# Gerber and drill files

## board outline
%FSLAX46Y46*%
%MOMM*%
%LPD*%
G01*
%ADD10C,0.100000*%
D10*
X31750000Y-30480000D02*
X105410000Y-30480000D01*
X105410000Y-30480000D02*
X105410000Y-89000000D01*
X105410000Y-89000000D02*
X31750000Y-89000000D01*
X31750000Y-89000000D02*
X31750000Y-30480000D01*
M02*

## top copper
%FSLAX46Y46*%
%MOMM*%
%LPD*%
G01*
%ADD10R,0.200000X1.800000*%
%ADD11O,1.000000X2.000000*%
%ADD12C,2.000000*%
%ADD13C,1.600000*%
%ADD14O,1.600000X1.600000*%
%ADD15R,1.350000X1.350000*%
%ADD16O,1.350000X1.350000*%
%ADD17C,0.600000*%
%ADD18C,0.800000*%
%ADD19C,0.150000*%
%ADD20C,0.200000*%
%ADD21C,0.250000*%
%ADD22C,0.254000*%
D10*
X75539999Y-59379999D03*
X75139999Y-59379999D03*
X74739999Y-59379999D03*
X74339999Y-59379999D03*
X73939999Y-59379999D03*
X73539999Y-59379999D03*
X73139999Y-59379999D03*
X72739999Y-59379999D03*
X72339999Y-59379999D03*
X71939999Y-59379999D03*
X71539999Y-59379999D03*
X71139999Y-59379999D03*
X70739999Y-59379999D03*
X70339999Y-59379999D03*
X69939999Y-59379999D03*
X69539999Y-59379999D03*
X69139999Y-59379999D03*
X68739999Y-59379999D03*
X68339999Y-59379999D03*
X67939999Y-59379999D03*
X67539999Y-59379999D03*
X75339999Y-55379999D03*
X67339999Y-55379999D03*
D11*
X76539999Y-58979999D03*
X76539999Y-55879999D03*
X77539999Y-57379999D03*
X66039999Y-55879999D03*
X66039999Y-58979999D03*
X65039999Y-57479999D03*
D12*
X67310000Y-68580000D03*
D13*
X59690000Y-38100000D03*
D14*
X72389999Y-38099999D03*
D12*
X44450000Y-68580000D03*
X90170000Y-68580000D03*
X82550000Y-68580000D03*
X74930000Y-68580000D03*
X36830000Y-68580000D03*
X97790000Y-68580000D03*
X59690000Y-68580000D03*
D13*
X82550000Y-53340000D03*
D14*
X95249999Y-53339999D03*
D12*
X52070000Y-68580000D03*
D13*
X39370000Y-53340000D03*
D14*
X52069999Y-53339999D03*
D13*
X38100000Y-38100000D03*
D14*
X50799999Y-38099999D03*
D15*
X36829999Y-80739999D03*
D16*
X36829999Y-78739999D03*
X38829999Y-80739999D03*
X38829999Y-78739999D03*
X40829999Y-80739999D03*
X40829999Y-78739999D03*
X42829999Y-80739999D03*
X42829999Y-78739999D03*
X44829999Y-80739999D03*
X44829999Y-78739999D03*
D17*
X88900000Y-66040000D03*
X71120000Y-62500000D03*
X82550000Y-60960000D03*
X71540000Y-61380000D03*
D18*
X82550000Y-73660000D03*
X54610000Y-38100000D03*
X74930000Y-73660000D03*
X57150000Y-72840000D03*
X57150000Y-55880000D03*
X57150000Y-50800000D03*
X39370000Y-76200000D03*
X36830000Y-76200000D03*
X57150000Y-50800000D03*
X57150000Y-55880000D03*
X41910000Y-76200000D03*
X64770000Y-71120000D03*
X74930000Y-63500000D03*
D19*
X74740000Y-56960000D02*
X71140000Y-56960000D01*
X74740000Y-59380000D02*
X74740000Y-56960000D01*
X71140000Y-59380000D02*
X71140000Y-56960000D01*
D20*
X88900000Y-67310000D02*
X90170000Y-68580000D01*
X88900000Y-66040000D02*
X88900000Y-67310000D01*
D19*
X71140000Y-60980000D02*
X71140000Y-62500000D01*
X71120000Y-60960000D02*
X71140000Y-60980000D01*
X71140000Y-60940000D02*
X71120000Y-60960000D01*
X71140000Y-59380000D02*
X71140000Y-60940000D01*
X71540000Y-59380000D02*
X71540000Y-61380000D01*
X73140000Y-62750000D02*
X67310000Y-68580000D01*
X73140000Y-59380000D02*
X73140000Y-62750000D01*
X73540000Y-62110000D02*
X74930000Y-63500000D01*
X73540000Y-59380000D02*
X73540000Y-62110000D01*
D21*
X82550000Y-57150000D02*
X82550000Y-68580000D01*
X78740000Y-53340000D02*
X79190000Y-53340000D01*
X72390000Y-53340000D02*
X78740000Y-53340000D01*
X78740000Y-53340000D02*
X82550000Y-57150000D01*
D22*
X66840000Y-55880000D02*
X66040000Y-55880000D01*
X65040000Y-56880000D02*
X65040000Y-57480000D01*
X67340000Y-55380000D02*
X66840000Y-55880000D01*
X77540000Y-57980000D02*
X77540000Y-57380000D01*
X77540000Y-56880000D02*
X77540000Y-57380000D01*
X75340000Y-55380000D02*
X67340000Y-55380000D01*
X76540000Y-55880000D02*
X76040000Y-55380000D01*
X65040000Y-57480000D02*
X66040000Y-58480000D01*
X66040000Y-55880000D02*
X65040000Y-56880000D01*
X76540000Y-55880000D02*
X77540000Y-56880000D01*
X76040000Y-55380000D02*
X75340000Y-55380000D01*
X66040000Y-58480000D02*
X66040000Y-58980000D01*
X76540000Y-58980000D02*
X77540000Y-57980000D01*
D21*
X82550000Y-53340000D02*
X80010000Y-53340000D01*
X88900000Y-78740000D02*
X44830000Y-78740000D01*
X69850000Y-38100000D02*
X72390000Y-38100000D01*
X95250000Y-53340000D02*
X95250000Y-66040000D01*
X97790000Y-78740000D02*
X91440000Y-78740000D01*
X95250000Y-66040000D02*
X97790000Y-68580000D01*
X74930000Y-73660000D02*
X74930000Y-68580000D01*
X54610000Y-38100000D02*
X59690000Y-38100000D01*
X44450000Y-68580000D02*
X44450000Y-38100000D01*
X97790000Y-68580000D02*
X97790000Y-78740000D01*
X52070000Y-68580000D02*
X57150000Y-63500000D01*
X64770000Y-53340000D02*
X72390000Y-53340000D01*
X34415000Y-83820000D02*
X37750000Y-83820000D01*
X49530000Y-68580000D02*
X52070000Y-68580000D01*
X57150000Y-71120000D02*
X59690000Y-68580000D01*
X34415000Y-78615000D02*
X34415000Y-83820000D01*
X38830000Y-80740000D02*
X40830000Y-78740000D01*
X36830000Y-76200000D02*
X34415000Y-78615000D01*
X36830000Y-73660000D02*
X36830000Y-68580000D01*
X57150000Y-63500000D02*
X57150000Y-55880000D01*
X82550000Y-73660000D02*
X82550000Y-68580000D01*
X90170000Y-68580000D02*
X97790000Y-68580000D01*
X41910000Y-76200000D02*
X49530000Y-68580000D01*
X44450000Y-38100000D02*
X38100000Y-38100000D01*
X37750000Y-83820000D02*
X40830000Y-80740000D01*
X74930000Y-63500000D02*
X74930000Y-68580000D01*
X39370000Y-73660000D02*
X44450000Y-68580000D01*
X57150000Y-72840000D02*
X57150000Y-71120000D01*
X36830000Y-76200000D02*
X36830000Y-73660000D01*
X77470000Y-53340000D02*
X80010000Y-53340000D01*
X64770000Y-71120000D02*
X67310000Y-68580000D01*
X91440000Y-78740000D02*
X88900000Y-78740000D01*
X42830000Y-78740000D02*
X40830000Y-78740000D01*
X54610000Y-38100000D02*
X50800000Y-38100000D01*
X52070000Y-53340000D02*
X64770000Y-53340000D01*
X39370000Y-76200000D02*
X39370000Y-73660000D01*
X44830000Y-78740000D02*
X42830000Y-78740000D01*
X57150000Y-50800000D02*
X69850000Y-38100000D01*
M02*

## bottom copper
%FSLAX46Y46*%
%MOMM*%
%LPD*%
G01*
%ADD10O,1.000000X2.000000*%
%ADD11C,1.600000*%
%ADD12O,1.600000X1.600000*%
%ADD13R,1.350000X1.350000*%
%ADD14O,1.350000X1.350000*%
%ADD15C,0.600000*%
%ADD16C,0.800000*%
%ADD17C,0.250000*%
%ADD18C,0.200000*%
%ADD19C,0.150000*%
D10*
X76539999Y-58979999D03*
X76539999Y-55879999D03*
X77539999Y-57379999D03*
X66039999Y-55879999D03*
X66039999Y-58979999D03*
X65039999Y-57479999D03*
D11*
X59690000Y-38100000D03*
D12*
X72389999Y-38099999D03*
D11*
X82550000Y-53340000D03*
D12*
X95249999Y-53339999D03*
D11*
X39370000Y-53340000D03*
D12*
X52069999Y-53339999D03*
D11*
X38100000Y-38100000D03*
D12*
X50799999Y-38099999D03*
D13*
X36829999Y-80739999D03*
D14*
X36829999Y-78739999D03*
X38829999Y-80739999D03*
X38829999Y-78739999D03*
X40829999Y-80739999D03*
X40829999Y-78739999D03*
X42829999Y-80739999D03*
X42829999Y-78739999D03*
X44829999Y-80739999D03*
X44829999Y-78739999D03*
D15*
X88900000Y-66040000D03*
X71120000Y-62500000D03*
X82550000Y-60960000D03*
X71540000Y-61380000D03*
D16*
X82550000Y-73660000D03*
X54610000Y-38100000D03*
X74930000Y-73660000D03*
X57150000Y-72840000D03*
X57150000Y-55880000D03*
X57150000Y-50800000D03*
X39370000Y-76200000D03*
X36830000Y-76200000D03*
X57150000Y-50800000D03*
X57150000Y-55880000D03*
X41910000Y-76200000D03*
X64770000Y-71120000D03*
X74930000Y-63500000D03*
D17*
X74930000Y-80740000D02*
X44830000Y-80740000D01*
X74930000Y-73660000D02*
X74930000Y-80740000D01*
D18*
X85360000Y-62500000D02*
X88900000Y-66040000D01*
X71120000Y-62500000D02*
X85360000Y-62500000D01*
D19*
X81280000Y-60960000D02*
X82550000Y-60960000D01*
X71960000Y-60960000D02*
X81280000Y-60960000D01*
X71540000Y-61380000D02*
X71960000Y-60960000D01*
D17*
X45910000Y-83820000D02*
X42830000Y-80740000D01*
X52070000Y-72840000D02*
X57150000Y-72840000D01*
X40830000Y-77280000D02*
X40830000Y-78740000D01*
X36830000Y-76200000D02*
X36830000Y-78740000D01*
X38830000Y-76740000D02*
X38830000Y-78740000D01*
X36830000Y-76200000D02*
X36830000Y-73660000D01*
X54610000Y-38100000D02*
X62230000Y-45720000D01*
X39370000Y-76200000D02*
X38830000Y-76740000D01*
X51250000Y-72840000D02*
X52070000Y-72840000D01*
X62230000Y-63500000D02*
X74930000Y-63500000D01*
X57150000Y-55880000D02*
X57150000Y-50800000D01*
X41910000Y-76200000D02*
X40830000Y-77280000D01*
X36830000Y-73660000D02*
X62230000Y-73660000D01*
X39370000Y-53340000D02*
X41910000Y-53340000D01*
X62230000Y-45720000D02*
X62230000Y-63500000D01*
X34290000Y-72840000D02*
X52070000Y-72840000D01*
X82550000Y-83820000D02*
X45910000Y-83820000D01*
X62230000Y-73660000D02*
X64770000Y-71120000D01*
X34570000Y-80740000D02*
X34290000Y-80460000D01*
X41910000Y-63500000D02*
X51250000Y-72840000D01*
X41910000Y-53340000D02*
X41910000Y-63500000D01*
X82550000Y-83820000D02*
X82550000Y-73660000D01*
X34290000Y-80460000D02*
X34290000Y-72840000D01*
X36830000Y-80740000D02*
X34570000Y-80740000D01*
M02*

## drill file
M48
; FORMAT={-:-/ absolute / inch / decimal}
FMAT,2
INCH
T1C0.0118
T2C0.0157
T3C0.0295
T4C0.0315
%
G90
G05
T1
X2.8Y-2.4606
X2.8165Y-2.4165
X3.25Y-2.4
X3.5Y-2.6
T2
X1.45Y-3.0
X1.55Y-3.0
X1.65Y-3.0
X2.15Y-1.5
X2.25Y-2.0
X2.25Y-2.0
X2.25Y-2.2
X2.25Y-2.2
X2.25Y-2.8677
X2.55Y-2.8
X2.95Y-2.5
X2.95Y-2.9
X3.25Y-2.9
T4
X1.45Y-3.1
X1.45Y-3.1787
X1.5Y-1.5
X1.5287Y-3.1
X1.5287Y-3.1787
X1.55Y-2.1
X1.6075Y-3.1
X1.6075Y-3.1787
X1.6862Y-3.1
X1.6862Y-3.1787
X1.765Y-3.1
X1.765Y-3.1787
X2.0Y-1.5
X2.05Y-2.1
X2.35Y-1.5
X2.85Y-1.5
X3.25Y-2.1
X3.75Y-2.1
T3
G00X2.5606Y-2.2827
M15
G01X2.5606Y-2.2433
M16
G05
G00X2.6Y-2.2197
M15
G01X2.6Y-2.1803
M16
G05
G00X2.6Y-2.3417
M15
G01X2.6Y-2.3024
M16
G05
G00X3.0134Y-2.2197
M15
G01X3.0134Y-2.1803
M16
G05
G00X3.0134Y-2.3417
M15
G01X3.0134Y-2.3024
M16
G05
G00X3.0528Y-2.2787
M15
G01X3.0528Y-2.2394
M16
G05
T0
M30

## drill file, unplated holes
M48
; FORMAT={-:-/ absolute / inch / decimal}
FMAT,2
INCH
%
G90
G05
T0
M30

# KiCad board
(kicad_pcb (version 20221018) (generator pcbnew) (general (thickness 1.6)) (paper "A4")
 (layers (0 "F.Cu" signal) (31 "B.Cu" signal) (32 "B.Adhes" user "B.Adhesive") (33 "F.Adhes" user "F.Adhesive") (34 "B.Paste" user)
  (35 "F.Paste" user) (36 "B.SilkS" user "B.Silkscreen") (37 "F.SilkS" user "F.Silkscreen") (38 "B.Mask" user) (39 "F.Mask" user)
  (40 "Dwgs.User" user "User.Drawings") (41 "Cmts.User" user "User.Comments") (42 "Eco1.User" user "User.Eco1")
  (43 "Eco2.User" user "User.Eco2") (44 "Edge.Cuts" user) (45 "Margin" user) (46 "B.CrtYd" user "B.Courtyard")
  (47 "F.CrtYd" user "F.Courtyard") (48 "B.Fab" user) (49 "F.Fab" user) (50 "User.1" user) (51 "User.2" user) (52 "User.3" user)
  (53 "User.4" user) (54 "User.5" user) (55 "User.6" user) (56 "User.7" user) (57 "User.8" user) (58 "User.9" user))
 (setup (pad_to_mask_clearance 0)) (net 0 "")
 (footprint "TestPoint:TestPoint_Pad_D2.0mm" (layer "F.Cu") (at 67.31 68.58)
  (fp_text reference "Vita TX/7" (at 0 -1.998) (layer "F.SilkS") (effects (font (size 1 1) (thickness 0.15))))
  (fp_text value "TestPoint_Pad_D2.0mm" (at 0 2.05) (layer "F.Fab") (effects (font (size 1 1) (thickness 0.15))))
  (pad "1" smd circle (at 0 0) (size 2 2) (layers "F.Cu" "F.Mask")))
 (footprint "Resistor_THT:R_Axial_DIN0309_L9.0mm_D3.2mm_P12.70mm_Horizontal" (layer "F.Cu") (at 59.69 38.1)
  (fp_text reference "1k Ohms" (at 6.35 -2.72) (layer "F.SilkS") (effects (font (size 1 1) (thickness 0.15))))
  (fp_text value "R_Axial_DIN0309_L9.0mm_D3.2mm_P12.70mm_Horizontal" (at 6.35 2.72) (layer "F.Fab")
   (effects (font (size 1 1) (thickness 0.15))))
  (pad "1" thru_hole circle (at 0 0) (size 1.6 1.6) (drill 0.8) (layers "*.Cu" "*.Mask"))
  (pad "2" thru_hole oval (at 12.7 0) (size 1.6 1.6) (drill 0.8) (layers "*.Cu" "*.Mask")))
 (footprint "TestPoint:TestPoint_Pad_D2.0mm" (layer "F.Cu") (at 44.45 68.58)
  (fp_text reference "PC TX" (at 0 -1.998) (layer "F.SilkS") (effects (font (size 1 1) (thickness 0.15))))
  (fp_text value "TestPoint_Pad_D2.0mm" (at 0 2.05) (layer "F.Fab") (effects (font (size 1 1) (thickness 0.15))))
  (pad "1" smd circle (at 0 0) (size 2 2) (layers "F.Cu" "F.Mask")))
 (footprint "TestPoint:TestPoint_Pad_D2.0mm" (layer "F.Cu") (at 90.17 68.58)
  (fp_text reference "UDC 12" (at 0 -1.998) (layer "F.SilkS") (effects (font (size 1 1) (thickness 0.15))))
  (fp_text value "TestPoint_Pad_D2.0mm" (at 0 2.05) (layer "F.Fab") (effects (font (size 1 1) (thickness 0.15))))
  (pad "1" smd circle (at 0 0) (size 2 2) (layers "F.Cu" "F.Mask")))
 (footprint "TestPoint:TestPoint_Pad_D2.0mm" (layer "F.Cu") (at 82.55 68.58)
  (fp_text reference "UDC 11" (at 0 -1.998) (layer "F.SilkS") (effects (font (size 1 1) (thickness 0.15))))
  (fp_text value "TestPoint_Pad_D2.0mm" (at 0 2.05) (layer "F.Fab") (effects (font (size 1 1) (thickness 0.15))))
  (pad "1" smd circle (at 0 0) (size 2 2) (layers "F.Cu" "F.Mask")))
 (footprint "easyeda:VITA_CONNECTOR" (layer "F.Cu") (at 76.54 58.98 180)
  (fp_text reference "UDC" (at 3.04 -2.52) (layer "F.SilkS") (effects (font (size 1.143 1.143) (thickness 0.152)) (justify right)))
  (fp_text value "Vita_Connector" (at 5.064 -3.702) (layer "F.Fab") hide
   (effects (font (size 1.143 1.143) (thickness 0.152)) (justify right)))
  (pad "1" smd rect (at 1 -0.4 180) (size 0.2 1.8) (layers "F.Cu" "F.Paste" "F.Mask"))
  (pad "2" smd rect (at 1.4 -0.4 180) (size 0.2 1.8) (layers "F.Cu" "F.Paste" "F.Mask"))
  (pad "3" smd rect (at 1.8 -0.4 180) (size 0.2 1.8) (layers "F.Cu" "F.Paste" "F.Mask"))
  (pad "4" smd rect (at 2.2 -0.4 180) (size 0.2 1.8) (layers "F.Cu" "F.Paste" "F.Mask"))
  (pad "5" smd rect (at 2.6 -0.4 180) (size 0.2 1.8) (layers "F.Cu" "F.Paste" "F.Mask"))
  (pad "6" smd rect (at 3 -0.4 180) (size 0.2 1.8) (layers "F.Cu" "F.Paste" "F.Mask"))
  (pad "7" smd rect (at 3.4 -0.4 180) (size 0.2 1.8) (layers "F.Cu" "F.Paste" "F.Mask"))
  (pad "8" smd rect (at 3.8 -0.4 180) (size 0.2 1.8) (layers "F.Cu" "F.Paste" "F.Mask"))
  (pad "9" smd rect (at 4.2 -0.4 180) (size 0.2 1.8) (layers "F.Cu" "F.Paste" "F.Mask"))
  (pad "10" smd rect (at 4.6 -0.4 180) (size 0.2 1.8) (layers "F.Cu" "F.Paste" "F.Mask"))
  (pad "11" smd rect (at 5 -0.4 180) (size 0.2 1.8) (layers "F.Cu" "F.Paste" "F.Mask"))
  (pad "12" smd rect (at 5.4 -0.4 180) (size 0.2 1.8) (layers "F.Cu" "F.Paste" "F.Mask"))
  (pad "13" smd rect (at 5.8 -0.4 180) (size 0.2 1.8) (layers "F.Cu" "F.Paste" "F.Mask"))
  (pad "14" smd rect (at 6.2 -0.4 180) (size 0.2 1.8) (layers "F.Cu" "F.Paste" "F.Mask"))
  (pad "15" smd rect (at 6.6 -0.4 180) (size 0.2 1.8) (layers "F.Cu" "F.Paste" "F.Mask"))
  (pad "16" smd rect (at 7 -0.4 180) (size 0.2 1.8) (layers "F.Cu" "F.Paste" "F.Mask"))
  (pad "17" smd rect (at 7.4 -0.4 180) (size 0.2 1.8) (layers "F.Cu" "F.Paste" "F.Mask"))
  (pad "18" smd rect (at 7.8 -0.4 180) (size 0.2 1.8) (layers "F.Cu" "F.Paste" "F.Mask"))
  (pad "19" smd rect (at 8.2 -0.4 180) (size 0.2 1.8) (layers "F.Cu" "F.Paste" "F.Mask"))
  (pad "20" smd rect (at 8.6 -0.4 180) (size 0.2 1.8) (layers "F.Cu" "F.Paste" "F.Mask"))
  (pad "21" smd rect (at 9 -0.4 180) (size 0.2 1.8) (layers "F.Cu" "F.Paste" "F.Mask"))
  (pad "22" smd rect (at 1.2 3.6 180) (size 0.2 1.8) (layers "F.Cu" "F.Paste" "F.Mask"))
  (pad "23" smd rect (at 9.2 3.6 180) (size 0.2 1.8) (layers "F.Cu" "F.Paste" "F.Mask"))
  (pad "24" thru_hole oval (at 0 0 180) (size 1 2) (drill oval 0.75 1.75) (layers "*.Cu" "*.Paste" "*.Mask"))
  (pad "25" thru_hole oval (at 0 3.1 180) (size 1 2) (drill oval 0.75 1.75) (layers "*.Cu" "*.Paste" "*.Mask"))
  (pad "26" thru_hole oval (at -1 1.6 180) (size 1 2) (drill oval 0.75 1.75) (layers "*.Cu" "*.Paste" "*.Mask"))
  (pad "27" thru_hole oval (at 10.5 3.1 180) (size 1 2) (drill oval 0.75 1.75) (layers "*.Cu" "*.Paste" "*.Mask"))
  (pad "28" thru_hole oval (at 10.5 0 180) (size 1 2) (drill oval 0.75 1.75) (layers "*.Cu" "*.Paste" "*.Mask"))
  (pad "29" thru_hole oval (at 11.5 1.5 180) (size 1 2) (drill oval 0.75 1.75) (layers "*.Cu" "*.Paste" "*.Mask")))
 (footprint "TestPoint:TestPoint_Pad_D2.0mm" (layer "F.Cu") (at 74.93 68.58)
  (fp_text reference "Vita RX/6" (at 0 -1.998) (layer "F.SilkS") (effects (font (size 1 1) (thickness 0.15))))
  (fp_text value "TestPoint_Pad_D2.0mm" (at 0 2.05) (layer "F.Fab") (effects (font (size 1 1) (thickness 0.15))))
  (pad "1" smd circle (at 0 0) (size 2 2) (layers "F.Cu" "F.Mask")))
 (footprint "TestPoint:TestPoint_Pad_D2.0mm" (layer "F.Cu") (at 36.83 68.58)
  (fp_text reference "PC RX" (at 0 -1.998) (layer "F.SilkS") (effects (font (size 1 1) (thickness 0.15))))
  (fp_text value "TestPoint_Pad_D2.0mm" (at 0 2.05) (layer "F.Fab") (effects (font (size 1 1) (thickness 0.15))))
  (pad "1" smd circle (at 0 0) (size 2 2) (layers "F.Cu" "F.Mask")))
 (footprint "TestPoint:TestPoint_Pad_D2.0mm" (layer "F.Cu") (at 97.79 68.58)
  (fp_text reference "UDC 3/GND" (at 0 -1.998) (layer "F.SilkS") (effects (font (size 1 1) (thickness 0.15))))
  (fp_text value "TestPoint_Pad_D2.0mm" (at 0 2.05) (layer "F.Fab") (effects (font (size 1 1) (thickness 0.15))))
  (pad "1" smd circle (at 0 0) (size 2 2) (layers "F.Cu" "F.Mask")))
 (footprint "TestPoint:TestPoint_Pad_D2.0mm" (layer "F.Cu") (at 59.69 68.58)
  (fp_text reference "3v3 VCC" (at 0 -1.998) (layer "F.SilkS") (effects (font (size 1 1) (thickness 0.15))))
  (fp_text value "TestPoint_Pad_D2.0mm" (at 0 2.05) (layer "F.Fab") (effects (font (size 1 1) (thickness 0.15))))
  (pad "1" smd circle (at 0 0) (size 2 2) (layers "F.Cu" "F.Mask")))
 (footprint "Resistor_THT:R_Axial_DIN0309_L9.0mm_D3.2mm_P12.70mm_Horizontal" (layer "F.Cu") (at 82.55 53.34)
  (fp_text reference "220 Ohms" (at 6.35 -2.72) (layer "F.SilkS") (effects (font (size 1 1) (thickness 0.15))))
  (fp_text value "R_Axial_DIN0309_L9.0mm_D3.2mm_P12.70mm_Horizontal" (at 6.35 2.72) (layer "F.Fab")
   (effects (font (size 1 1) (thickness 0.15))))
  (pad "1" thru_hole circle (at 0 0) (size 1.6 1.6) (drill 0.8) (layers "*.Cu" "*.Mask"))
  (pad "2" thru_hole oval (at 12.7 0) (size 1.6 1.6) (drill 0.8) (layers "*.Cu" "*.Mask")))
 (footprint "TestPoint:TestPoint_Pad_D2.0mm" (layer "F.Cu") (at 52.07 68.58)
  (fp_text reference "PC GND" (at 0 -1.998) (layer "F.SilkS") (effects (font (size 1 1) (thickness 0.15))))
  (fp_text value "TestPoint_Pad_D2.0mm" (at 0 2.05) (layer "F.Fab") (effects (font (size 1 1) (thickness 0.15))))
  (pad "1" smd circle (at 0 0) (size 2 2) (layers "F.Cu" "F.Mask")))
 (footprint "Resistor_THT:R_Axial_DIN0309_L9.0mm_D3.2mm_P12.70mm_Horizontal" (layer "F.Cu") (at 39.37 53.34)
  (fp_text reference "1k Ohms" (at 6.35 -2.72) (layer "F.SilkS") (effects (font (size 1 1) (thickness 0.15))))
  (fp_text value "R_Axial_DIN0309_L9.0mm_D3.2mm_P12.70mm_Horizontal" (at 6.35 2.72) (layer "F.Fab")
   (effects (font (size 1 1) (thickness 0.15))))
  (pad "1" thru_hole circle (at 0 0) (size 1.6 1.6) (drill 0.8) (layers "*.Cu" "*.Mask"))
  (pad "2" thru_hole oval (at 12.7 0) (size 1.6 1.6) (drill 0.8) (layers "*.Cu" "*.Mask")))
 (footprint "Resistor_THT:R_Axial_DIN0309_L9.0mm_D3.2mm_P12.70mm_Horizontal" (layer "F.Cu") (at 38.1 38.1)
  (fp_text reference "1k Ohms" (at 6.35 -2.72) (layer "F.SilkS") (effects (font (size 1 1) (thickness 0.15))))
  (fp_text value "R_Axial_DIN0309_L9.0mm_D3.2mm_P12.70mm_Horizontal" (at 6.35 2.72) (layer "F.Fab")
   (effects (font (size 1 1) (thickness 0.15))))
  (pad "1" thru_hole circle (at 0 0) (size 1.6 1.6) (drill 0.8) (layers "*.Cu" "*.Mask"))
  (pad "2" thru_hole oval (at 12.7 0) (size 1.6 1.6) (drill 0.8) (layers "*.Cu" "*.Mask")))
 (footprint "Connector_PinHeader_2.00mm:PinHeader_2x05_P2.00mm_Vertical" (layer "F.Cu") (at 36.83 80.74 90)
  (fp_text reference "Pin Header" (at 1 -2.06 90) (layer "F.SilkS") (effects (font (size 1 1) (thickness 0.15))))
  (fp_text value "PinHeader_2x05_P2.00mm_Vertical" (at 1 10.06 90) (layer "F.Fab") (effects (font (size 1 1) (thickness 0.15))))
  (pad "1" thru_hole rect (at 0 0 90) (size 1.35 1.35) (drill 0.8) (layers "*.Cu" "*.Mask"))
  (pad "2" thru_hole oval (at 2 0 90) (size 1.35 1.35) (drill 0.8) (layers "*.Cu" "*.Mask"))
  (pad "3" thru_hole oval (at 0 2 90) (size 1.35 1.35) (drill 0.8) (layers "*.Cu" "*.Mask"))
  (pad "4" thru_hole oval (at 2 2 90) (size 1.35 1.35) (drill 0.8) (layers "*.Cu" "*.Mask"))
  (pad "5" thru_hole oval (at 0 4 90) (size 1.35 1.35) (drill 0.8) (layers "*.Cu" "*.Mask"))
  (pad "6" thru_hole oval (at 2 4 90) (size 1.35 1.35) (drill 0.8) (layers "*.Cu" "*.Mask"))
  (pad "7" thru_hole oval (at 0 6 90) (size 1.35 1.35) (drill 0.8) (layers "*.Cu" "*.Mask"))
  (pad "8" thru_hole oval (at 2 6 90) (size 1.35 1.35) (drill 0.8) (layers "*.Cu" "*.Mask"))
  (pad "9" thru_hole oval (at 0 8 90) (size 1.35 1.35) (drill 0.8) (layers "*.Cu" "*.Mask"))
  (pad "10" thru_hole oval (at 2 8 90) (size 1.35 1.35) (drill 0.8) (layers "*.Cu" "*.Mask")))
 (gr_rect (start 31.75 30.48) (end 105.41 89) (stroke (width 0.1) (type default)) (fill none) (layer "Edge.Cuts"))
 (segment (start 82.55 53.34) (end 80.01 53.34) (width 0.25) (layer "F.Cu") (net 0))
 (segment (start 88.9 78.74) (end 44.83 78.74) (width 0.25) (layer "F.Cu") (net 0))
 (segment (start 69.85 38.1) (end 72.39 38.1) (width 0.25) (layer "F.Cu") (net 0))
 (segment (start 95.25 53.34) (end 95.25 66.04) (width 0.25) (layer "F.Cu") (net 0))
 (segment (start 97.79 78.74) (end 91.44 78.74) (width 0.25) (layer "F.Cu") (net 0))
 (segment (start 66.04 58.48) (end 66.04 58.98) (width 0.254) (layer "F.Cu") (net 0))
 (segment (start 95.25 66.04) (end 97.79 68.58) (width 0.25) (layer "F.Cu") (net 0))
 (segment (start 74.93 73.66) (end 74.93 68.58) (width 0.25) (layer "F.Cu") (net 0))
 (segment (start 77.54 57.98) (end 77.54 57.38) (width 0.254) (layer "F.Cu") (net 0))
 (segment (start 54.61 38.1) (end 59.69 38.1) (width 0.25) (layer "F.Cu") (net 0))
 (segment (start 71.14 59.38) (end 71.14 60.94) (width 0.15) (layer "F.Cu") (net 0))
 (segment (start 44.45 68.58) (end 44.45 38.1) (width 0.25) (layer "F.Cu") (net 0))
 (segment (start 97.79 68.58) (end 97.79 78.74) (width 0.25) (layer "F.Cu") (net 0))
 (segment (start 67.34 55.38) (end 66.84 55.88) (width 0.254) (layer "F.Cu") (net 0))
 (segment (start 52.07 68.58) (end 57.15 63.5) (width 0.25) (layer "F.Cu") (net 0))
 (segment (start 64.77 53.34) (end 72.39 53.34) (width 0.25) (layer "F.Cu") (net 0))
 (segment (start 34.415 83.82) (end 37.75 83.82) (width 0.25) (layer "F.Cu") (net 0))
 (segment (start 73.54 59.38) (end 73.54 62.11) (width 0.15) (layer "F.Cu") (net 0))
 (segment (start 73.14 59.38) (end 73.14 62.75) (width 0.15) (layer "F.Cu") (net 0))
 (segment (start 65.04 57.48) (end 66.04 58.48) (width 0.254) (layer "F.Cu") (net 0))
 (segment (start 49.53 68.58) (end 52.07 68.58) (width 0.25) (layer "F.Cu") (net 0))
 (segment (start 57.15 71.12) (end 59.69 68.58) (width 0.25) (layer "F.Cu") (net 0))
 (segment (start 34.415 78.615) (end 34.415 83.82) (width 0.25) (layer "F.Cu") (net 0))
 (segment (start 38.83 80.74) (end 40.83 78.74) (width 0.25) (layer "F.Cu") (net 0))
 (segment (start 66.84 55.88) (end 66.04 55.88) (width 0.254) (layer "F.Cu") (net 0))
 (segment (start 36.83 76.2) (end 34.415 78.615) (width 0.25) (layer "F.Cu") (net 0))
 (segment (start 36.83 73.66) (end 36.83 68.58) (width 0.25) (layer "F.Cu") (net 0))
 (segment (start 71.14 60.98) (end 71.14 62.5) (width 0.15) (layer "F.Cu") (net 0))
 (segment (start 57.15 63.5) (end 57.15 55.88) (width 0.25) (layer "F.Cu") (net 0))
 (segment (start 82.55 73.66) (end 82.55 68.58) (width 0.25) (layer "F.Cu") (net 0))
 (segment (start 90.17 68.58) (end 97.79 68.58) (width 0.25) (layer "F.Cu") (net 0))
 (segment (start 65.04 56.88) (end 65.04 57.48) (width 0.254) (layer "F.Cu") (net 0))
 (segment (start 77.54 56.88) (end 77.54 57.38) (width 0.254) (layer "F.Cu") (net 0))
 (segment (start 76.54 58.98) (end 77.54 57.98) (width 0.254) (layer "F.Cu") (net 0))
 (segment (start 41.91 76.2) (end 49.53 68.58) (width 0.25) (layer "F.Cu") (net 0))
 (segment (start 71.54 59.38) (end 71.54 61.38) (width 0.15) (layer "F.Cu") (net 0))
 (segment (start 44.45 38.1) (end 38.1 38.1) (width 0.25) (layer "F.Cu") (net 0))
 (segment (start 78.74 53.34) (end 79.19 53.34) (width 0.25) (layer "F.Cu") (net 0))
 (segment (start 37.75 83.82) (end 40.83 80.74) (width 0.25) (layer "F.Cu") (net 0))
 (segment (start 74.93 63.5) (end 74.93 68.58) (width 0.25) (layer "F.Cu") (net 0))
 (segment (start 73.54 62.11) (end 74.93 63.5) (width 0.15) (layer "F.Cu") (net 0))
 (segment (start 39.37 73.66) (end 44.45 68.58) (width 0.25) (layer "F.Cu") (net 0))
 (segment (start 57.15 72.84) (end 57.15 71.12) (width 0.25) (layer "F.Cu") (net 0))
 (segment (start 88.9 66.04) (end 88.9 67.31) (width 0.2) (layer "F.Cu") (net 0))
 (segment (start 36.83 76.2) (end 36.83 73.66) (width 0.25) (layer "F.Cu") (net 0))
 (segment (start 77.47 53.34) (end 80.01 53.34) (width 0.25) (layer "F.Cu") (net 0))
 (segment (start 64.77 71.12) (end 67.31 68.58) (width 0.25) (layer "F.Cu") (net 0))
 (segment (start 76.04 55.38) (end 75.34 55.38) (width 0.254) (layer "F.Cu") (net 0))
 (segment (start 91.44 78.74) (end 88.9 78.74) (width 0.25) (layer "F.Cu") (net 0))
 (segment (start 71.14 60.94) (end 71.12 60.96) (width 0.15) (layer "F.Cu") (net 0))
 (segment (start 82.55 57.15) (end 82.55 68.58) (width 0.25) (layer "F.Cu") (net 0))
 (segment (start 42.83 78.74) (end 40.83 78.74) (width 0.25) (layer "F.Cu") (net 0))
 (segment (start 72.39 53.34) (end 78.74 53.34) (width 0.25) (layer "F.Cu") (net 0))
 (segment (start 54.61 38.1) (end 50.8 38.1) (width 0.25) (layer "F.Cu") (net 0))
 (segment (start 52.07 53.34) (end 64.77 53.34) (width 0.25) (layer "F.Cu") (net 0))
 (segment (start 76.54 55.88) (end 77.54 56.88) (width 0.254) (layer "F.Cu") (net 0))
 (segment (start 66.04 55.88) (end 65.04 56.88) (width 0.254) (layer "F.Cu") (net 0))
 (segment (start 39.37 76.2) (end 39.37 73.66) (width 0.25) (layer "F.Cu") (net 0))
 (segment (start 44.83 78.74) (end 42.83 78.74) (width 0.25) (layer "F.Cu") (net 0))
 (segment (start 57.15 50.8) (end 69.85 38.1) (width 0.25) (layer "F.Cu") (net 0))
 (segment (start 78.74 53.34) (end 82.55 57.15) (width 0.25) (layer "F.Cu") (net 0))
 (segment (start 75.34 55.38) (end 67.34 55.38) (width 0.254) (layer "F.Cu") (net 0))
 (segment (start 76.54 55.88) (end 76.04 55.38) (width 0.254) (layer "F.Cu") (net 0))
 (segment (start 71.12 60.96) (end 71.14 60.98) (width 0.15) (layer "F.Cu") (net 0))
 (segment (start 88.9 67.31) (end 90.17 68.58) (width 0.2) (layer "F.Cu") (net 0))
 (segment (start 74.74 56.96) (end 71.14 56.96) (width 0.15) (layer "F.Cu") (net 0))
 (segment (start 74.74 59.38) (end 74.74 56.96) (width 0.15) (layer "F.Cu") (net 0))
 (segment (start 71.14 59.38) (end 71.14 56.96) (width 0.15) (layer "F.Cu") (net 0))
 (segment (start 73.14 62.75) (end 67.31 68.58) (width 0.15) (layer "F.Cu") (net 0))
 (via (at 82.55 73.66) (size 0.8) (drill 0.4) (layers "F.Cu" "B.Cu") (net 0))
 (via (at 71.54 61.38) (size 0.6) (drill 0.3) (layers "F.Cu" "B.Cu") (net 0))
 (via (at 54.61 38.1) (size 0.8) (drill 0.4) (layers "F.Cu" "B.Cu") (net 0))
 (via (at 74.93 73.66) (size 0.8) (drill 0.4) (layers "F.Cu" "B.Cu") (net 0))
 (via (at 57.15 72.84) (size 0.8) (drill 0.4) (layers "F.Cu" "B.Cu") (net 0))
 (via (at 57.15 55.88) (size 0.8) (drill 0.4) (layers "F.Cu" "B.Cu") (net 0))
 (via (at 71.12 62.5) (size 0.6) (drill 0.3) (layers "F.Cu" "B.Cu") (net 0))
 (via (at 57.15 50.8) (size 0.8) (drill 0.4) (layers "F.Cu" "B.Cu") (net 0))
 (via (at 39.37 76.2) (size 0.8) (drill 0.4) (layers "F.Cu" "B.Cu") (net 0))
 (via (at 88.9 66.04) (size 0.6) (drill 0.3) (layers "F.Cu" "B.Cu") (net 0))
 (via (at 36.83 76.2) (size 0.8) (drill 0.4) (layers "F.Cu" "B.Cu") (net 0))
 (via (at 57.15 50.8) (size 0.8) (drill 0.4) (layers "F.Cu" "B.Cu") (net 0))
 (via (at 57.15 55.88) (size 0.8) (drill 0.4) (layers "F.Cu" "B.Cu") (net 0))
 (via (at 41.91 76.2) (size 0.8) (drill 0.4) (layers "F.Cu" "B.Cu") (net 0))
 (via (at 64.77 71.12) (size 0.8) (drill 0.4) (layers "F.Cu" "B.Cu") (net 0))
 (via (at 82.55 60.96) (size 0.6) (drill 0.3) (layers "F.Cu" "B.Cu") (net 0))
 (via (at 74.93 63.5) (size 0.8) (drill 0.4) (layers "F.Cu" "B.Cu") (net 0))
 (segment (start 45.91 83.82) (end 42.83 80.74) (width 0.25) (layer "B.Cu") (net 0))
 (segment (start 52.07 72.84) (end 57.15 72.84) (width 0.25) (layer "B.Cu") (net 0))
 (segment (start 40.83 77.28) (end 40.83 78.74) (width 0.25) (layer "B.Cu") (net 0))
 (segment (start 36.83 76.2) (end 36.83 78.74) (width 0.25) (layer "B.Cu") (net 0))
 (segment (start 38.83 76.74) (end 38.83 78.74) (width 0.25) (layer "B.Cu") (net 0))
 (segment (start 74.93 80.74) (end 44.83 80.74) (width 0.25) (layer "B.Cu") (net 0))
 (segment (start 36.83 76.2) (end 36.83 73.66) (width 0.25) (layer "B.Cu") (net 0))
 (segment (start 54.61 38.1) (end 62.23 45.72) (width 0.25) (layer "B.Cu") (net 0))
 (segment (start 39.37 76.2) (end 38.83 76.74) (width 0.25) (layer "B.Cu") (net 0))
 (segment (start 51.25 72.84) (end 52.07 72.84) (width 0.25) (layer "B.Cu") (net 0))
 (segment (start 62.23 63.5) (end 74.93 63.5) (width 0.25) (layer "B.Cu") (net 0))
 (segment (start 57.15 55.88) (end 57.15 50.8) (width 0.25) (layer "B.Cu") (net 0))
 (segment (start 81.28 60.96) (end 82.55 60.96) (width 0.15) (layer "B.Cu") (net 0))
 (segment (start 41.91 76.2) (end 40.83 77.28) (width 0.25) (layer "B.Cu") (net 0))
 (segment (start 85.36 62.5) (end 88.9 66.04) (width 0.2) (layer "B.Cu") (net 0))
 (segment (start 71.96 60.96) (end 81.28 60.96) (width 0.15) (layer "B.Cu") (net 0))
 (segment (start 36.83 73.66) (end 62.23 73.66) (width 0.25) (layer "B.Cu") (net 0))
 (segment (start 74.93 73.66) (end 74.93 80.74) (width 0.25) (layer "B.Cu") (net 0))
 (segment (start 39.37 53.34) (end 41.91 53.34) (width 0.25) (layer "B.Cu") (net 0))
 (segment (start 62.23 45.72) (end 62.23 63.5) (width 0.25) (layer "B.Cu") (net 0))
 (segment (start 34.29 72.84) (end 52.07 72.84) (width 0.25) (layer "B.Cu") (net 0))
 (segment (start 71.54 61.38) (end 71.96 60.96) (width 0.15) (layer "B.Cu") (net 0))
 (segment (start 82.55 83.82) (end 45.91 83.82) (width 0.25) (layer "B.Cu") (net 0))
 (segment (start 62.23 73.66) (end 64.77 71.12) (width 0.25) (layer "B.Cu") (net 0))
 (segment (start 34.57 80.74) (end 34.29 80.46) (width 0.25) (layer "B.Cu") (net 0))
 (segment (start 41.91 63.5) (end 51.25 72.84) (width 0.25) (layer "B.Cu") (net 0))
 (segment (start 41.91 53.34) (end 41.91 63.5) (width 0.25) (layer "B.Cu") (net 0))
 (segment (start 82.55 83.82) (end 82.55 73.66) (width 0.25) (layer "B.Cu") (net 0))
 (segment (start 34.29 80.46) (end 34.29 72.84) (width 0.25) (layer "B.Cu") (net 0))
 (segment (start 36.83 80.74) (end 34.57 80.74) (width 0.25) (layer "B.Cu") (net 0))
 (segment (start 71.12 62.5) (end 85.36 62.5) (width 0.2) (layer "B.Cu") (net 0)))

